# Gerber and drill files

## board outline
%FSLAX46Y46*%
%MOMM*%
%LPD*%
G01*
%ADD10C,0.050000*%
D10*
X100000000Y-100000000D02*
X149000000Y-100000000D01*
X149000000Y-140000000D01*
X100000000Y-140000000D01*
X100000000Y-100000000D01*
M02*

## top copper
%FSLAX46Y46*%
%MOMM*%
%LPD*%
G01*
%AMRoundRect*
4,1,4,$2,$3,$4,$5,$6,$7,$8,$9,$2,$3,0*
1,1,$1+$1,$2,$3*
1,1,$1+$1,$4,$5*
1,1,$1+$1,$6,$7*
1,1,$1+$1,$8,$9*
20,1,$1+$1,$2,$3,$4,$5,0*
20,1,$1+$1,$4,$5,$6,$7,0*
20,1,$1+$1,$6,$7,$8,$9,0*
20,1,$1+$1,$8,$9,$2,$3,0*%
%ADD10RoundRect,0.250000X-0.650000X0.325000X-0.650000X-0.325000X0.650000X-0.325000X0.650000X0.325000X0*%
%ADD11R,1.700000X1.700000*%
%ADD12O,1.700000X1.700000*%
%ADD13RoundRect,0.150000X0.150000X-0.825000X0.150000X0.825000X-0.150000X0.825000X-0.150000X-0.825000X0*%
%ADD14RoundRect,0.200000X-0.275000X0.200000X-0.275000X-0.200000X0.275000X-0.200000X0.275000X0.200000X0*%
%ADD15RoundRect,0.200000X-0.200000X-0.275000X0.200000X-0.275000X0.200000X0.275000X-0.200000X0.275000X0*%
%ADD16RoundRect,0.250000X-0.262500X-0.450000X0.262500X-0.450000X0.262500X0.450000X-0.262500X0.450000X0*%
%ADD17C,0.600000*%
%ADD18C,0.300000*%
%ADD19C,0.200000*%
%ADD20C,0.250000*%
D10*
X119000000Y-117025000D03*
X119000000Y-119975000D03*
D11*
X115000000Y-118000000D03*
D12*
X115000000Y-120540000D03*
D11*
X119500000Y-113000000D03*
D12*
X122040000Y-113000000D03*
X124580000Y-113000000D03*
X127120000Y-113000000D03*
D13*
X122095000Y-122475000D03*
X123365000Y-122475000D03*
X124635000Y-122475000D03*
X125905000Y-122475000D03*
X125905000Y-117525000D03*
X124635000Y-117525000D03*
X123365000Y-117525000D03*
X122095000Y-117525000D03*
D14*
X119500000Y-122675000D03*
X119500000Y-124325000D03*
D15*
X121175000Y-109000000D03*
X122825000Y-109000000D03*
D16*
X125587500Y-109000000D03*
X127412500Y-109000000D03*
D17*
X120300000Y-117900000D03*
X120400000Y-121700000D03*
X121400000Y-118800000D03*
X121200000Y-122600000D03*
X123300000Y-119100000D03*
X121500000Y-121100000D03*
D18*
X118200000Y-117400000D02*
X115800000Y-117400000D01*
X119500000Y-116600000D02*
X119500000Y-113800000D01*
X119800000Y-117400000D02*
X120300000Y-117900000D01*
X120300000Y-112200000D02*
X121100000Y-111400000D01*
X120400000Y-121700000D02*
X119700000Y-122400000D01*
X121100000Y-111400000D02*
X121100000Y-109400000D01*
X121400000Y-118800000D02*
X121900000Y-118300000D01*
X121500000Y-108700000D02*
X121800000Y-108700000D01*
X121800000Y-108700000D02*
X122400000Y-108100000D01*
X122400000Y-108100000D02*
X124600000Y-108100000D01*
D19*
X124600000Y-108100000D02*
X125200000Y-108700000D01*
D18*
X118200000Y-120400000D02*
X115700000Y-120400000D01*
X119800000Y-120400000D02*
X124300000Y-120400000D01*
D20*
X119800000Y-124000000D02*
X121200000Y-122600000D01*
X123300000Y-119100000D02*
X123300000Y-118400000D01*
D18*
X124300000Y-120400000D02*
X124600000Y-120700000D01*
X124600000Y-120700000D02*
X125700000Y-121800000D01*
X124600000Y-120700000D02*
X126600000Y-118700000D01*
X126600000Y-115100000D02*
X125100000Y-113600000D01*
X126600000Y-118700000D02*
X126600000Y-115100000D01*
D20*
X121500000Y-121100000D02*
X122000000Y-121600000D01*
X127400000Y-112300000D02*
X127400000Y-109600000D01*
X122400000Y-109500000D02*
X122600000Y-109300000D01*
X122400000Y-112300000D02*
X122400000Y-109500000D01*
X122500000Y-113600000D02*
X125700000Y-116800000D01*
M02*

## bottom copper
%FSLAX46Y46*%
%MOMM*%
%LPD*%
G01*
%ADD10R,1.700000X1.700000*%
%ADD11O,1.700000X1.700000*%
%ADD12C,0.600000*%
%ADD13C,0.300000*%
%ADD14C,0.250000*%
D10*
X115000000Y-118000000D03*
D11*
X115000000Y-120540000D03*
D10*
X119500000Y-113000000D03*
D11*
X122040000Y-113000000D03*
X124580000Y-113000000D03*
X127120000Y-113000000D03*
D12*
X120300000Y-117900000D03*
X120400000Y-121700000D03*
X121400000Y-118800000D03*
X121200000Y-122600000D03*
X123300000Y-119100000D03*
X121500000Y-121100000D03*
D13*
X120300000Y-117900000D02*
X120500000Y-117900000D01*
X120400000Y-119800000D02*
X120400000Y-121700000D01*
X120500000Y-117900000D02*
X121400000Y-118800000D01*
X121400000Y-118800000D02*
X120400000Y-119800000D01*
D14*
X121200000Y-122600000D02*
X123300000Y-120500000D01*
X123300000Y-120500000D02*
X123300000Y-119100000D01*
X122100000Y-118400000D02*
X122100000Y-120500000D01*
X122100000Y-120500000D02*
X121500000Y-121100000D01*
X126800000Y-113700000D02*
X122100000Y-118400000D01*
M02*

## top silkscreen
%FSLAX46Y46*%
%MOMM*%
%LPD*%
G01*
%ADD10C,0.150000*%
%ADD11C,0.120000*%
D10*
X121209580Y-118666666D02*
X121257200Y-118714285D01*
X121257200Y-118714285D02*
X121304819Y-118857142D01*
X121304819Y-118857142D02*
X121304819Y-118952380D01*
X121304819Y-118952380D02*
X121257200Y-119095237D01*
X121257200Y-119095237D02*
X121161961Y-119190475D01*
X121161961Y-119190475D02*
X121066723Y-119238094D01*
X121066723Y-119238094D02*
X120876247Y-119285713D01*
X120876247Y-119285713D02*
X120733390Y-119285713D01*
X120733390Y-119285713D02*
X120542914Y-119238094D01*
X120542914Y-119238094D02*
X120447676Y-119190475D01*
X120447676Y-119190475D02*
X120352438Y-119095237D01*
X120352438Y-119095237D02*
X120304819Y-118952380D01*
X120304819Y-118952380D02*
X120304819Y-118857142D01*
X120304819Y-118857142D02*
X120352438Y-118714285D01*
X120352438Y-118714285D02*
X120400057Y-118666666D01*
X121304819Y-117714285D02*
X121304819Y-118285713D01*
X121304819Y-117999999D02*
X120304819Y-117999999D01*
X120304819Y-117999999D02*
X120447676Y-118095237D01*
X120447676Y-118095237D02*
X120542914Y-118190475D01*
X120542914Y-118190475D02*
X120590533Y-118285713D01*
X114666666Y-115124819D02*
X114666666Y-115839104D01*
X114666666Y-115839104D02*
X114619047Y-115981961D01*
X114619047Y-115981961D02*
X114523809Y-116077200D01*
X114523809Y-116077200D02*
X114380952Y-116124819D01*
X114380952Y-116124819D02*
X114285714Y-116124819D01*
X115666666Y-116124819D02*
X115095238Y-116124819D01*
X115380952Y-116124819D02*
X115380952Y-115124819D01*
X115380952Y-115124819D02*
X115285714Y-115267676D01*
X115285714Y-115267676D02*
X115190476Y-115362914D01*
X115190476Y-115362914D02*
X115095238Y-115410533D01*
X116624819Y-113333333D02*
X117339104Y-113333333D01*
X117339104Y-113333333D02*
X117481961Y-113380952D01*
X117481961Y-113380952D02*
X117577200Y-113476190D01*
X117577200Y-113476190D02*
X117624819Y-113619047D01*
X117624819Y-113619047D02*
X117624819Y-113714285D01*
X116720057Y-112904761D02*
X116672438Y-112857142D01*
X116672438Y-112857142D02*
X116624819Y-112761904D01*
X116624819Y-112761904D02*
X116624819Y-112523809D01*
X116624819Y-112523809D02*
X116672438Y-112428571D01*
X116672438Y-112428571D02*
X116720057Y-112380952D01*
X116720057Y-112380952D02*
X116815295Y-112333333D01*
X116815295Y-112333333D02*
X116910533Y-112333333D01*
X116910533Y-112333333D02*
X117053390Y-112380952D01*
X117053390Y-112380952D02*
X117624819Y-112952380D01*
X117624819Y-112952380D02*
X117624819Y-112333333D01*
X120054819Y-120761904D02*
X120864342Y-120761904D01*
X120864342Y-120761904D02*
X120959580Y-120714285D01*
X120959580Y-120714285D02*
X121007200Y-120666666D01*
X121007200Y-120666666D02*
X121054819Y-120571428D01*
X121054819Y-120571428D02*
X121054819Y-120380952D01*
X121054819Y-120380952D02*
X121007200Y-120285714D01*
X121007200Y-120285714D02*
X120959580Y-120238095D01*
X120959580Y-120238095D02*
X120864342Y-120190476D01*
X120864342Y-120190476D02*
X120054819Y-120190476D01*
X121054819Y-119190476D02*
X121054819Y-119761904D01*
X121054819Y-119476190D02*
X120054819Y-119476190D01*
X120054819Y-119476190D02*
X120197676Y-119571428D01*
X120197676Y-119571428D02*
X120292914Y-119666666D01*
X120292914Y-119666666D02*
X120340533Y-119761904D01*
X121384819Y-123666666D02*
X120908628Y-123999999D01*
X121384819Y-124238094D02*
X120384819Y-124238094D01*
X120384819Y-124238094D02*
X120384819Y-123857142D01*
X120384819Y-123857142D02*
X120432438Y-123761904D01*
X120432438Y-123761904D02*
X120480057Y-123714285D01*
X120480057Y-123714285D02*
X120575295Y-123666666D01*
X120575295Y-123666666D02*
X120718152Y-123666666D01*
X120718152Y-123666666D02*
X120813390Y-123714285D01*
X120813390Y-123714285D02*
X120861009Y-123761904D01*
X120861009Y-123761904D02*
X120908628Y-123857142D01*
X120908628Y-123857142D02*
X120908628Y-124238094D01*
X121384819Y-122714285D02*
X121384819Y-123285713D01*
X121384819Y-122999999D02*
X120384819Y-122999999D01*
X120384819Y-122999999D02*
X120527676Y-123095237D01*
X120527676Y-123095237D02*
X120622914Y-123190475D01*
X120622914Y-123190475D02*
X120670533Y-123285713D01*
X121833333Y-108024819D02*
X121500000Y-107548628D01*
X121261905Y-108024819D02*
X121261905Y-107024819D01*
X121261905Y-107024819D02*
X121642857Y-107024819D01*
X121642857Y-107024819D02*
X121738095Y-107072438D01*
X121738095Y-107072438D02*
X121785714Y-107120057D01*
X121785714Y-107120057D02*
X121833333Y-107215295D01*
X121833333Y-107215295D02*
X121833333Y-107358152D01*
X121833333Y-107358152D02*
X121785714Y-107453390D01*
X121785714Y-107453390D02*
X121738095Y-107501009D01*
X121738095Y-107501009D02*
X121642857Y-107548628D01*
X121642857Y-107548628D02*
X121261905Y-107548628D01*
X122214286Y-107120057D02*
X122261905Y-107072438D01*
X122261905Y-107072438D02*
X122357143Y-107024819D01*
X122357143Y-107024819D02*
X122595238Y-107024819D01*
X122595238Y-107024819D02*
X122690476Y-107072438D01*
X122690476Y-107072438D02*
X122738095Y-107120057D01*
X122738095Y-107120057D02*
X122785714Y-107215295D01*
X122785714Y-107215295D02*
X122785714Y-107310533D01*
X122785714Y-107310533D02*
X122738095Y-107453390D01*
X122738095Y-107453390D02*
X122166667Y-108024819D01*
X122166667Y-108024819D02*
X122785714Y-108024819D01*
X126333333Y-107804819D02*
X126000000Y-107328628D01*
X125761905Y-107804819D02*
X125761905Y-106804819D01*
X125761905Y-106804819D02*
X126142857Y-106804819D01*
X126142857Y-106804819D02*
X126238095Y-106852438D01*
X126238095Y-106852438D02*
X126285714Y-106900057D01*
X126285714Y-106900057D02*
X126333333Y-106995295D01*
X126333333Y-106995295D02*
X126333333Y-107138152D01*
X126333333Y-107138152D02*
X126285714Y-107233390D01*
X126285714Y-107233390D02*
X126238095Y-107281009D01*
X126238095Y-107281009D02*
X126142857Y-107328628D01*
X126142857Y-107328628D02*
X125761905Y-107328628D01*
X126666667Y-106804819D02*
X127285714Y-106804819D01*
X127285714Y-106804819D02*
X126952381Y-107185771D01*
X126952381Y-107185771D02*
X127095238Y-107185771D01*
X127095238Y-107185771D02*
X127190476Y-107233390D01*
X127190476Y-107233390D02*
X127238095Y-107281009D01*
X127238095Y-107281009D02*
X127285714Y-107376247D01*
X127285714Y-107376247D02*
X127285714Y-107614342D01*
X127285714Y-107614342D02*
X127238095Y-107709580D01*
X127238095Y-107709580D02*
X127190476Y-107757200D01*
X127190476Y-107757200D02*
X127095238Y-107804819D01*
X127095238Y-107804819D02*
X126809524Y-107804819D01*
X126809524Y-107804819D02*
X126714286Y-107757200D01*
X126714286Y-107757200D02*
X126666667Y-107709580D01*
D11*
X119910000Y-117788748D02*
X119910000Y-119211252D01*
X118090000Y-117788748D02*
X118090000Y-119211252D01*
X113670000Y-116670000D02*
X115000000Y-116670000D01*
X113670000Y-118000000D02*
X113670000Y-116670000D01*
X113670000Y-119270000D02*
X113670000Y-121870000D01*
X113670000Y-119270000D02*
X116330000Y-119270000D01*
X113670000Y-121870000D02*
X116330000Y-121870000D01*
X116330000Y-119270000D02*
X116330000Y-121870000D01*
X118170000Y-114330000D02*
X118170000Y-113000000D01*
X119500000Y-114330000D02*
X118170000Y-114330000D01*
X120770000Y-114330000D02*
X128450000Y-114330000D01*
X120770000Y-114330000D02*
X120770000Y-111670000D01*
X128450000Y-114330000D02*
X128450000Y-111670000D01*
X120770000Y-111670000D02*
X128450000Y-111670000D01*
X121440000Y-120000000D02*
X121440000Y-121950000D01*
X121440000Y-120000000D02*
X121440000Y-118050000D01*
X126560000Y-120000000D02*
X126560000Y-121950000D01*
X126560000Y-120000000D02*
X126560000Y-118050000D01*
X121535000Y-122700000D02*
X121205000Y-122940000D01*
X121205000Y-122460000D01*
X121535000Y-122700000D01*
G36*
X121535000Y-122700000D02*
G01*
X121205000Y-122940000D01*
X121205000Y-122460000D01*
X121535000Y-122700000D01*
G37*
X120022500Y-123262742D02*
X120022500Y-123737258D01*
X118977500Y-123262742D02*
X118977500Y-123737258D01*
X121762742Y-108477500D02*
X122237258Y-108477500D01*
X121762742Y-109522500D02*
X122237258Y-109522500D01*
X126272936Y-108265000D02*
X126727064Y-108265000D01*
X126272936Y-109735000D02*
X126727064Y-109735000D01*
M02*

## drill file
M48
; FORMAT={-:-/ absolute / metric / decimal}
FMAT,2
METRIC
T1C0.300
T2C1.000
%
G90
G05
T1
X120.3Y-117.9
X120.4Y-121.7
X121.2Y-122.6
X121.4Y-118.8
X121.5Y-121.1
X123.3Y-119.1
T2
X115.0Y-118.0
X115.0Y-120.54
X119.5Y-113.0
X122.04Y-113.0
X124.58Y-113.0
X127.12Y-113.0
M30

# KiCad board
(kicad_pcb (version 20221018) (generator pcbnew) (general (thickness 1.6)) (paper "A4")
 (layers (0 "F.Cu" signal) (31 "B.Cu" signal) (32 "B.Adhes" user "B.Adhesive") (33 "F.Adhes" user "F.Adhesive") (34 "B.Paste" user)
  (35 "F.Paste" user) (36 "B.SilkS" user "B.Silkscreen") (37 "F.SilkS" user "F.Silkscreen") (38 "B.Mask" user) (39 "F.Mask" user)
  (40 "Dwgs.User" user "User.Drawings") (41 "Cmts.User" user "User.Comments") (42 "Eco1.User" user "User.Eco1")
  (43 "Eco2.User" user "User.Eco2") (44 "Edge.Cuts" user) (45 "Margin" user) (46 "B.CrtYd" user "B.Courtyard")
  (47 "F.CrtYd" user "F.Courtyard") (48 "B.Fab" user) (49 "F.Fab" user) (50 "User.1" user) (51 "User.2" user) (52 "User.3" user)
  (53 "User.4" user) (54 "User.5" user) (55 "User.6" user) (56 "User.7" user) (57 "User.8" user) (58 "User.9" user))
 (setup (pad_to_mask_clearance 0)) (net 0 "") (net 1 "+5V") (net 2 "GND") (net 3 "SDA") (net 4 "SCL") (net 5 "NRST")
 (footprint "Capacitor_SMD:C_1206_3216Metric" (layer "F.Cu") (at 119 118.5 -90)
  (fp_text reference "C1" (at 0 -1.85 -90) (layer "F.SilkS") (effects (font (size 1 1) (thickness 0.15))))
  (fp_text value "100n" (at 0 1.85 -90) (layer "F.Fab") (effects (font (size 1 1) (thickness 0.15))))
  (fp_line (start -0.711252 -0.91) (end 0.711252 -0.91) (stroke (width 0.12) (type solid)) (layer "F.SilkS"))
  (fp_line (start -0.711252 0.91) (end 0.711252 0.91) (stroke (width 0.12) (type solid)) (layer "F.SilkS"))
  (pad "1" smd roundrect (at -1.475 0 270) (size 1.15 1.8) (layers "F.Cu" "F.Paste" "F.Mask") (roundrect_rratio 0.217391) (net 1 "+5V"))
  (pad "2" smd roundrect (at 1.475 0 270) (size 1.15 1.8) (layers "F.Cu" "F.Paste" "F.Mask") (roundrect_rratio 0.217391) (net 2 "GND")))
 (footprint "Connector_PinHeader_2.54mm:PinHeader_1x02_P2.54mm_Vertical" (layer "F.Cu") (at 115 118)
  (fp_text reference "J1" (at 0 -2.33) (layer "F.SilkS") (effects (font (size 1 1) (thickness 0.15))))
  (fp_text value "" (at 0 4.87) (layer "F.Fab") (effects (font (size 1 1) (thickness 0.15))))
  (fp_line (start -1.33 -1.33) (end 0 -1.33) (stroke (width 0.12) (type solid)) (layer "F.SilkS"))
  (fp_line (start -1.33 0) (end -1.33 -1.33) (stroke (width 0.12) (type solid)) (layer "F.SilkS"))
  (fp_line (start -1.33 1.27) (end -1.33 3.87) (stroke (width 0.12) (type solid)) (layer "F.SilkS"))
  (fp_line (start -1.33 1.27) (end 1.33 1.27) (stroke (width 0.12) (type solid)) (layer "F.SilkS"))
  (fp_line (start -1.33 3.87) (end 1.33 3.87) (stroke (width 0.12) (type solid)) (layer "F.SilkS"))
  (fp_line (start 1.33 1.27) (end 1.33 3.87) (stroke (width 0.12) (type solid)) (layer "F.SilkS"))
  (pad "1" thru_hole rect (at 0 0) (size 1.7 1.7) (drill 1) (layers "*.Cu" "*.Mask") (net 1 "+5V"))
  (pad "2" thru_hole oval (at 0 2.54) (size 1.7 1.7) (drill 1) (layers "*.Cu" "*.Mask") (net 2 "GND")))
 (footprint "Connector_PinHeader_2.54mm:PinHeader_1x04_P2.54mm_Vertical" (layer "F.Cu") (at 119.5 113 90)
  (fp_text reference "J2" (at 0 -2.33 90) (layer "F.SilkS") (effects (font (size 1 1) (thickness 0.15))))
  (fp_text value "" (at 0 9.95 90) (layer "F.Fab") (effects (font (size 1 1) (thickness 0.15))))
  (fp_line (start -1.33 -1.33) (end 0 -1.33) (stroke (width 0.12) (type solid)) (layer "F.SilkS"))
  (fp_line (start -1.33 0) (end -1.33 -1.33) (stroke (width 0.12) (type solid)) (layer "F.SilkS"))
  (fp_line (start -1.33 1.27) (end -1.33 8.95) (stroke (width 0.12) (type solid)) (layer "F.SilkS"))
  (fp_line (start -1.33 1.27) (end 1.33 1.27) (stroke (width 0.12) (type solid)) (layer "F.SilkS"))
  (fp_line (start -1.33 8.95) (end 1.33 8.95) (stroke (width 0.12) (type solid)) (layer "F.SilkS"))
  (fp_line (start 1.33 1.27) (end 1.33 8.95) (stroke (width 0.12) (type solid)) (layer "F.SilkS"))
  (pad "1" thru_hole rect (at 0 0 90) (size 1.7 1.7) (drill 1) (layers "*.Cu" "*.Mask") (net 1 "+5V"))
  (pad "2" thru_hole oval (at 0 2.54 90) (size 1.7 1.7) (drill 1) (layers "*.Cu" "*.Mask") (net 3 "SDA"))
  (pad "3" thru_hole oval (at 0 5.08 90) (size 1.7 1.7) (drill 1) (layers "*.Cu" "*.Mask") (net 2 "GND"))
  (pad "4" thru_hole oval (at 0 7.62 90) (size 1.7 1.7) (drill 1) (layers "*.Cu" "*.Mask") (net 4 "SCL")))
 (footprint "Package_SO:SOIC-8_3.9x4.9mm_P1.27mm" (layer "F.Cu") (at 124 120 90)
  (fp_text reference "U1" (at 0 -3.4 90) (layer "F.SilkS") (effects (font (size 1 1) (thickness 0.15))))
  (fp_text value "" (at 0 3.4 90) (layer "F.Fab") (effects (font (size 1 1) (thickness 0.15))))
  (fp_line (start 0 -2.56) (end -1.95 -2.56) (stroke (width 0.12) (type solid)) (layer "F.SilkS"))
  (fp_line (start 0 -2.56) (end 1.95 -2.56) (stroke (width 0.12) (type solid)) (layer "F.SilkS"))
  (fp_line (start 0 2.56) (end -1.95 2.56) (stroke (width 0.12) (type solid)) (layer "F.SilkS"))
  (fp_line (start 0 2.56) (end 1.95 2.56) (stroke (width 0.12) (type solid)) (layer "F.SilkS"))
  (fp_poly
   (pts (xy -2.7 -2.465) (xy -2.94 -2.795) (xy -2.46 -2.795) (xy -2.7 -2.465)) (stroke (width 0.12) (type solid)) (fill solid)
   (layer "F.SilkS"))
  (pad "1" smd roundrect (at -2.475 -1.905 90) (size 1.95 0.6) (layers "F.Cu" "F.Paste" "F.Mask") (roundrect_rratio 0.25) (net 4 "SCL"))
  (pad "2" smd roundrect (at -2.475 -0.635 90) (size 1.95 0.6) (layers "F.Cu" "F.Paste" "F.Mask") (roundrect_rratio 0.25))
  (pad "3" smd roundrect (at -2.475 0.635 90) (size 1.95 0.6) (layers "F.Cu" "F.Paste" "F.Mask") (roundrect_rratio 0.25))
  (pad "4" smd roundrect (at -2.475 1.905 90) (size 1.95 0.6) (layers "F.Cu" "F.Paste" "F.Mask") (roundrect_rratio 0.25) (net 2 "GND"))
  (pad "5" smd roundrect (at 2.475 1.905 90) (size 1.95 0.6) (layers "F.Cu" "F.Paste" "F.Mask") (roundrect_rratio 0.25) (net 3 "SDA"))
  (pad "6" smd roundrect (at 2.475 0.635 90) (size 1.95 0.6) (layers "F.Cu" "F.Paste" "F.Mask") (roundrect_rratio 0.25))
  (pad "7" smd roundrect (at 2.475 -0.635 90) (size 1.95 0.6) (layers "F.Cu" "F.Paste" "F.Mask") (roundrect_rratio 0.25) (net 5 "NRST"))
  (pad "8" smd roundrect (at 2.475 -1.905 90) (size 1.95 0.6) (layers "F.Cu" "F.Paste" "F.Mask") (roundrect_rratio 0.25) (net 1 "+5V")))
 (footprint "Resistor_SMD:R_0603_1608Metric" (layer "F.Cu") (at 119.5 123.5 -90)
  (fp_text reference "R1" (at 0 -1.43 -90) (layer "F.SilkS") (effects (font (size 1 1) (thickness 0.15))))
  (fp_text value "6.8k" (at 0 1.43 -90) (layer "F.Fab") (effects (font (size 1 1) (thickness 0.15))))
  (fp_line (start -0.237258 -0.5225) (end 0.237258 -0.5225) (stroke (width 0.12) (type solid)) (layer "F.SilkS"))
  (fp_line (start -0.237258 0.5225) (end 0.237258 0.5225) (stroke (width 0.12) (type solid)) (layer "F.SilkS"))
  (pad "1" smd roundrect (at -0.825 0 270) (size 0.8 0.95) (layers "F.Cu" "F.Paste" "F.Mask") (roundrect_rratio 0.25) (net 1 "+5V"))
  (pad "2" smd roundrect (at 0.825 0 270) (size 0.8 0.95) (layers "F.Cu" "F.Paste" "F.Mask") (roundrect_rratio 0.25) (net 5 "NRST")))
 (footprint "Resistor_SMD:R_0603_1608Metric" (layer "F.Cu") (at 122 109)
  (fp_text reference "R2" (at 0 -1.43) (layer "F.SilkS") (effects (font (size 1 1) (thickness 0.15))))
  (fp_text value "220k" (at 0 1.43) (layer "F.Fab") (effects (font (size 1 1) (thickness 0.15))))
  (fp_line (start -0.237258 -0.5225) (end 0.237258 -0.5225) (stroke (width 0.12) (type solid)) (layer "F.SilkS"))
  (fp_line (start -0.237258 0.5225) (end 0.237258 0.5225) (stroke (width 0.12) (type solid)) (layer "F.SilkS"))
  (pad "1" smd roundrect (at -0.825 0) (size 0.8 0.95) (layers "F.Cu" "F.Paste" "F.Mask") (roundrect_rratio 0.25) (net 1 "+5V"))
  (pad "2" smd roundrect (at 0.825 0) (size 0.8 0.95) (layers "F.Cu" "F.Paste" "F.Mask") (roundrect_rratio 0.25) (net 3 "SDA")))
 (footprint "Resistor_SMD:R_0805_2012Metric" (layer "F.Cu") (at 126.5 109)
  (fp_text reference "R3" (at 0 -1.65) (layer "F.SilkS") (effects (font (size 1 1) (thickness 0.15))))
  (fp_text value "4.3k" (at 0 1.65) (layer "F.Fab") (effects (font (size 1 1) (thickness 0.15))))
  (fp_line (start -0.227064 -0.735) (end 0.227064 -0.735) (stroke (width 0.12) (type solid)) (layer "F.SilkS"))
  (fp_line (start -0.227064 0.735) (end 0.227064 0.735) (stroke (width 0.12) (type solid)) (layer "F.SilkS"))
  (pad "1" smd roundrect (at -0.9125 0) (size 1.025 1.4) (layers "F.Cu" "F.Paste" "F.Mask") (roundrect_rratio 0.243902) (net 1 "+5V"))
  (pad "2" smd roundrect (at 0.9125 0) (size 1.025 1.4) (layers "F.Cu" "F.Paste" "F.Mask") (roundrect_rratio 0.243902) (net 4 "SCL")))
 (gr_rect (start 100 100) (end 149 140) (stroke (width 0.05) (type default)) (fill none) (layer "Edge.Cuts"))
 (segment (start 118.2 117.4) (end 115.8 117.4) (width 0.3) (layer "F.Cu") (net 1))
 (segment (start 119.5 116.6) (end 119.5 113.8) (width 0.3) (layer "F.Cu") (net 1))
 (segment (start 119.8 117.4) (end 120.3 117.9) (width 0.3) (layer "F.Cu") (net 1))
 (segment (start 120.3 112.2) (end 121.1 111.4) (width 0.3) (layer "F.Cu") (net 1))
 (segment (start 120.4 121.7) (end 119.7 122.4) (width 0.3) (layer "F.Cu") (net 1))
 (segment (start 121.1 111.4) (end 121.1 109.4) (width 0.3) (layer "F.Cu") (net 1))
 (segment (start 121.4 118.8) (end 121.9 118.3) (width 0.3) (layer "F.Cu") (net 1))
 (segment (start 121.5 108.7) (end 121.8 108.7) (width 0.3) (layer "F.Cu") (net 1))
 (segment (start 121.8 108.7) (end 122.4 108.1) (width 0.3) (layer "F.Cu") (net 1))
 (segment (start 122.4 108.1) (end 124.6 108.1) (width 0.3) (layer "F.Cu") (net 1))
 (segment (start 124.6 108.1) (end 125.2 108.7) (width 0.2) (layer "F.Cu") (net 1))
 (via (at 120.3 117.9) (size 0.6) (drill 0.3) (layers "F.Cu" "B.Cu") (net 1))
 (via (at 120.4 121.7) (size 0.6) (drill 0.3) (layers "F.Cu" "B.Cu") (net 1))
 (via (at 121.4 118.8) (size 0.6) (drill 0.3) (layers "F.Cu" "B.Cu") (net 1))
 (segment (start 118.2 120.4) (end 115.7 120.4) (width 0.3) (layer "F.Cu") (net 2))
 (segment (start 119.8 120.4) (end 124.3 120.4) (width 0.3) (layer "F.Cu") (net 2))
 (segment (start 119.8 124) (end 121.2 122.6) (width 0.25) (layer "F.Cu") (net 5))
 (segment (start 120.3 117.9) (end 120.5 117.9) (width 0.3) (layer "B.Cu") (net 1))
 (segment (start 120.4 119.8) (end 120.4 121.7) (width 0.3) (layer "B.Cu") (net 1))
 (segment (start 120.5 117.9) (end 121.4 118.8) (width 0.3) (layer "B.Cu") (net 1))
 (segment (start 121.4 118.8) (end 120.4 119.8) (width 0.3) (layer "B.Cu") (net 1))
 (segment (start 123.3 119.1) (end 123.3 118.4) (width 0.25) (layer "F.Cu") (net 5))
 (segment (start 124.3 120.4) (end 124.6 120.7) (width 0.3) (layer "F.Cu") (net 2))
 (segment (start 124.6 120.7) (end 125.7 121.8) (width 0.3) (layer "F.Cu") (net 2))
 (segment (start 124.6 120.7) (end 126.6 118.7) (width 0.3) (layer "F.Cu") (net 2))
 (segment (start 126.6 115.1) (end 125.1 113.6) (width 0.3) (layer "F.Cu") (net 2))
 (segment (start 126.6 118.7) (end 126.6 115.1) (width 0.3) (layer "F.Cu") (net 2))
 (via (at 121.2 122.6) (size 0.6) (drill 0.3) (layers "F.Cu" "B.Cu") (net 5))
 (via (at 123.3 119.1) (size 0.6) (drill 0.3) (layers "F.Cu" "B.Cu") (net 5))
 (segment (start 121.2 122.6) (end 123.3 120.5) (width 0.25) (layer "B.Cu") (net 5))
 (segment (start 121.5 121.1) (end 122 121.6) (width 0.25) (layer "F.Cu") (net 4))
 (segment (start 123.3 120.5) (end 123.3 119.1) (width 0.25) (layer "B.Cu") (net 5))
 (segment (start 127.4 112.3) (end 127.4 109.6) (width 0.25) (layer "F.Cu") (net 4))
 (via (at 121.5 121.1) (size 0.6) (drill 0.3) (layers "F.Cu" "B.Cu") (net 4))
 (segment (start 122.1 118.4) (end 122.1 120.5) (width 0.25) (layer "B.Cu") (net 4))
 (segment (start 122.1 120.5) (end 121.5 121.1) (width 0.25) (layer "B.Cu") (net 4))
 (segment (start 122.4 109.5) (end 122.6 109.3) (width 0.25) (layer "F.Cu") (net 3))
 (segment (start 122.4 112.3) (end 122.4 109.5) (width 0.25) (layer "F.Cu") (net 3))
 (segment (start 122.5 113.6) (end 125.7 116.8) (width 0.25) (layer "F.Cu") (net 3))
 (segment (start 126.8 113.7) (end 122.1 118.4) (width 0.25) (layer "B.Cu") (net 4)))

